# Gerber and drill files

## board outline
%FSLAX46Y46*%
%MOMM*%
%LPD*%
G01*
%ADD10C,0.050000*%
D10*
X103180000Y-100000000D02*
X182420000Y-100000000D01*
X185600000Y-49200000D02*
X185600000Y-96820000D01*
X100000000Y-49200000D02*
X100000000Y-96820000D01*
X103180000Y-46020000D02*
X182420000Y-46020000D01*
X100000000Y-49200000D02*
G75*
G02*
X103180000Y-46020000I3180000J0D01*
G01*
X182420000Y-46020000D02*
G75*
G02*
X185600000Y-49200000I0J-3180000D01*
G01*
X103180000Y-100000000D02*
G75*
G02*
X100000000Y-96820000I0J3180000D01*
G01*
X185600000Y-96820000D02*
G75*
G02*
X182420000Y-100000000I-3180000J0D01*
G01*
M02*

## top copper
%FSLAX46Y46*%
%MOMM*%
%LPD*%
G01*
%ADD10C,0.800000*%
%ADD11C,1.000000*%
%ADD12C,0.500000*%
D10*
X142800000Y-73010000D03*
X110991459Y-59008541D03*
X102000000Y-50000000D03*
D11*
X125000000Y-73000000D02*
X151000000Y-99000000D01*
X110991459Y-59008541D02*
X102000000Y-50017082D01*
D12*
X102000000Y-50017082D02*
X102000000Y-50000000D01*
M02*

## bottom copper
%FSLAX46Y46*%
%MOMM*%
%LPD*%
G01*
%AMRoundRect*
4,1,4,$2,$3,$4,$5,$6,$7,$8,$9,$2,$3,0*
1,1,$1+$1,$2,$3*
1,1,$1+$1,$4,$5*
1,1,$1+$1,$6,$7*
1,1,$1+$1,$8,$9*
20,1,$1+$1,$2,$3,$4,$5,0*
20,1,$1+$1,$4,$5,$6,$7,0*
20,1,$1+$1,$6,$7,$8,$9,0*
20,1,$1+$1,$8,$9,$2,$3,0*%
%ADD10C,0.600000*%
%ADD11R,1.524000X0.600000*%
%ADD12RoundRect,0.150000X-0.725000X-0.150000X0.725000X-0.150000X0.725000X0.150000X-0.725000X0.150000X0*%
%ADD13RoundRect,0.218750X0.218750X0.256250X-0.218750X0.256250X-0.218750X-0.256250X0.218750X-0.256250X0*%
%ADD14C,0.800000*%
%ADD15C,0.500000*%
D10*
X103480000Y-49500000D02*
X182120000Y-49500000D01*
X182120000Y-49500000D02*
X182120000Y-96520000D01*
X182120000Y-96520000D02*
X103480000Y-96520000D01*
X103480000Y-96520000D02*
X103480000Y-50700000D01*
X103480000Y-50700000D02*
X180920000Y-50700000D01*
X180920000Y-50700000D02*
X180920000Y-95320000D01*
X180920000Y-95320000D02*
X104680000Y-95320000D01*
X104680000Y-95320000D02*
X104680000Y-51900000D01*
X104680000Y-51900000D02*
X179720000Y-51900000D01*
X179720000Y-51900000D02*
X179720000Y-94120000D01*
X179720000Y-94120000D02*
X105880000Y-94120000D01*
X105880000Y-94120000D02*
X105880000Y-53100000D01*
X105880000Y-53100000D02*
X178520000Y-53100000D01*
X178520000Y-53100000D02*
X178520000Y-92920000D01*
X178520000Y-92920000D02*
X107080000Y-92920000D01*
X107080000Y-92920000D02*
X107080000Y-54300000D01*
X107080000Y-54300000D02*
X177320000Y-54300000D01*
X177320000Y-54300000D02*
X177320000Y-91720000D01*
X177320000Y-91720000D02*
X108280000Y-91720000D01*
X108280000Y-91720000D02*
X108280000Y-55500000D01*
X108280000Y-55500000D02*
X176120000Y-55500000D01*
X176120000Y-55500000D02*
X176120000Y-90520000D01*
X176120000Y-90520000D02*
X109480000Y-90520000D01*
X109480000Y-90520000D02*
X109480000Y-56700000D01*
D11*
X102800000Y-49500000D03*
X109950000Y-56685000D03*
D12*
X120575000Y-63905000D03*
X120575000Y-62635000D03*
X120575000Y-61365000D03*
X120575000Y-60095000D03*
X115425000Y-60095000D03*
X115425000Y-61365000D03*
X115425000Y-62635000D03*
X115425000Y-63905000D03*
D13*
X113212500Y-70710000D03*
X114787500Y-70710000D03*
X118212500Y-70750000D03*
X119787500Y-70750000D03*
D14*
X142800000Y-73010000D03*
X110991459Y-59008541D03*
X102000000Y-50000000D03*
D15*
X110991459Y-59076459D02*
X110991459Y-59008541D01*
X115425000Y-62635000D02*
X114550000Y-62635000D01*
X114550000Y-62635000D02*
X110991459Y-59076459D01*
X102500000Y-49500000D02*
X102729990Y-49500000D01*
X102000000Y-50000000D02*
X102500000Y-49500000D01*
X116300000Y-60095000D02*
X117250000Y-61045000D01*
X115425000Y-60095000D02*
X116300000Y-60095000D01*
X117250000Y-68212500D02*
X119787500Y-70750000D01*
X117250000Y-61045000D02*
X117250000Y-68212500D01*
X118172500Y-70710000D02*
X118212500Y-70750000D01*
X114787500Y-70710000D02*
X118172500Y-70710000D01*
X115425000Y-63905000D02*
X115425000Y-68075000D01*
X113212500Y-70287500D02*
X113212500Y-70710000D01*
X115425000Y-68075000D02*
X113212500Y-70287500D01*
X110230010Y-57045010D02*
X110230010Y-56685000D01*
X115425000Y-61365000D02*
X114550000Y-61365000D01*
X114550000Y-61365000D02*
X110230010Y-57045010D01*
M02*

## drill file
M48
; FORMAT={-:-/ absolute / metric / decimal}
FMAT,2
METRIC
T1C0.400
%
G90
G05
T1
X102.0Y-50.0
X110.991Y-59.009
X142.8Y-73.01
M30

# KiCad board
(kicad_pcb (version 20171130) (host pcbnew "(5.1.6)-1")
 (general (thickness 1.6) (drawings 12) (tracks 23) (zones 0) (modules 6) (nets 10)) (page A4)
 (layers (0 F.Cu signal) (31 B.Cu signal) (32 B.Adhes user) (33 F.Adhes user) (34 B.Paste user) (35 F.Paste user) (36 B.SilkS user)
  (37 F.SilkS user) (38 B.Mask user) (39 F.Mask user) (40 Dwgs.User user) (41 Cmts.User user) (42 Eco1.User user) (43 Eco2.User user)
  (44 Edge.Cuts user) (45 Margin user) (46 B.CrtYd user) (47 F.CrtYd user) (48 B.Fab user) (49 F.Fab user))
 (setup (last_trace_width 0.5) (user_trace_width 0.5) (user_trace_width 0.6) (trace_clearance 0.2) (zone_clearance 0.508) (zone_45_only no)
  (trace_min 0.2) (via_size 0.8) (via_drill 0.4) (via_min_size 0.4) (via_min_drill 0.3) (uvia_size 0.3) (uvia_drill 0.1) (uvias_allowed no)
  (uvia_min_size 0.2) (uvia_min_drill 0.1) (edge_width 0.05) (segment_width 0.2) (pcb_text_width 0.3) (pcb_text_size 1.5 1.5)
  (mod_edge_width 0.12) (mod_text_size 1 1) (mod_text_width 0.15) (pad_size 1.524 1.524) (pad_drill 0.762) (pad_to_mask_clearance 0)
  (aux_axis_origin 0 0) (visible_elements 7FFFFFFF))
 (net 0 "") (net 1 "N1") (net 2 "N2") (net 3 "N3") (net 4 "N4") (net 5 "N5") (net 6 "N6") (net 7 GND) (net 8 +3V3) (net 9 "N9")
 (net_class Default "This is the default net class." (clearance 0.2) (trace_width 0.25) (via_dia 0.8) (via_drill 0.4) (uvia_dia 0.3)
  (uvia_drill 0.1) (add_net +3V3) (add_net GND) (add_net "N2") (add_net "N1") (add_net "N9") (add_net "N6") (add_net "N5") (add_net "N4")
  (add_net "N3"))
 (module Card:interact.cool (layer F.Cu) (at 118 66 45)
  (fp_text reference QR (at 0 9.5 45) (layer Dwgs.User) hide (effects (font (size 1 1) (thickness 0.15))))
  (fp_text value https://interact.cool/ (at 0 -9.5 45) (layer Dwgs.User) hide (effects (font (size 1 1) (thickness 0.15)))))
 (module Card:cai (layer F.Cu) (at 150 73 270)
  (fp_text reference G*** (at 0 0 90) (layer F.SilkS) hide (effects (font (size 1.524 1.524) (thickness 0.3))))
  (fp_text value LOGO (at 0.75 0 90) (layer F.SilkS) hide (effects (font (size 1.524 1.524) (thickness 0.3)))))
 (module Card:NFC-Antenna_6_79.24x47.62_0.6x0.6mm (layer B.Cu) (at 142.8 73.01)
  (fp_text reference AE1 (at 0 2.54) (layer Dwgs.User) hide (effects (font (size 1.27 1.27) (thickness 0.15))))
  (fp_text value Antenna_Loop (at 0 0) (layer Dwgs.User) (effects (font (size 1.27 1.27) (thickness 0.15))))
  (fp_line (start -39.32 -23.51) (end 39.32 -23.51) (layer B.Cu) (width 0.6))
  (fp_line (start 39.32 -23.51) (end 39.32 23.51) (layer B.Cu) (width 0.6))
  (fp_line (start 39.32 23.51) (end -39.32 23.51) (layer B.Cu) (width 0.6))
  (fp_line (start -39.32 23.51) (end -39.32 -22.31) (layer B.Cu) (width 0.6))
  (fp_line (start -39.32 -22.31) (end 38.12 -22.31) (layer B.Cu) (width 0.6))
  (fp_line (start 38.12 -22.31) (end 38.12 22.31) (layer B.Cu) (width 0.6))
  (fp_line (start 38.12 22.31) (end -38.12 22.31) (layer B.Cu) (width 0.6))
  (fp_line (start -38.12 22.31) (end -38.12 -21.11) (layer B.Cu) (width 0.6))
  (fp_line (start -38.12 -21.11) (end 36.92 -21.11) (layer B.Cu) (width 0.6))
  (fp_line (start 36.92 -21.11) (end 36.92 21.11) (layer B.Cu) (width 0.6))
  (fp_line (start 36.92 21.11) (end -36.92 21.11) (layer B.Cu) (width 0.6))
  (fp_line (start -36.92 21.11) (end -36.92 -19.91) (layer B.Cu) (width 0.6))
  (fp_line (start -36.92 -19.91) (end 35.72 -19.91) (layer B.Cu) (width 0.6))
  (fp_line (start 35.72 -19.91) (end 35.72 19.91) (layer B.Cu) (width 0.6))
  (fp_line (start 35.72 19.91) (end -35.72 19.91) (layer B.Cu) (width 0.6))
  (fp_line (start -35.72 19.91) (end -35.72 -18.71) (layer B.Cu) (width 0.6))
  (fp_line (start -35.72 -18.71) (end 34.52 -18.71) (layer B.Cu) (width 0.6))
  (fp_line (start 34.52 -18.71) (end 34.52 18.71) (layer B.Cu) (width 0.6))
  (fp_line (start 34.52 18.71) (end -34.52 18.71) (layer B.Cu) (width 0.6))
  (fp_line (start -34.52 18.71) (end -34.52 -17.51) (layer B.Cu) (width 0.6))
  (fp_line (start -34.52 -17.51) (end 33.32 -17.51) (layer B.Cu) (width 0.6))
  (fp_line (start 33.32 -17.51) (end 33.32 17.51) (layer B.Cu) (width 0.6))
  (fp_line (start 33.32 17.51) (end -33.32 17.51) (layer B.Cu) (width 0.6))
  (fp_line (start -33.32 17.51) (end -33.32 -16.31) (layer B.Cu) (width 0.6))
  (pad 2 smd rect (at -40 -23.51) (size 1.524 0.6) (layers B.Cu) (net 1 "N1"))
  (pad 1 smd rect (at -32.85 -16.325) (size 1.524 0.6) (layers B.Cu) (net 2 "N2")))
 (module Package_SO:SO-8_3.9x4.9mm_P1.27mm (layer B.Cu) (at 118 62)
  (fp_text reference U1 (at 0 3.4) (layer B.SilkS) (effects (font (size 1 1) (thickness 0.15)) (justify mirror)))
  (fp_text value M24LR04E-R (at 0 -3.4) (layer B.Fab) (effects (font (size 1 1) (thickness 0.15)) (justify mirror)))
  (pad 8 smd roundrect (at 2.575 1.905) (size 1.75 0.6) (layers B.Cu B.Paste B.Mask) (roundrect_rratio 0.25) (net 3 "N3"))
  (pad 7 smd roundrect (at 2.575 0.635) (size 1.75 0.6) (layers B.Cu B.Paste B.Mask) (roundrect_rratio 0.25) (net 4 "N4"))
  (pad 6 smd roundrect (at 2.575 -0.635) (size 1.75 0.6) (layers B.Cu B.Paste B.Mask) (roundrect_rratio 0.25) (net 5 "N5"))
  (pad 5 smd roundrect (at 2.575 -1.905) (size 1.75 0.6) (layers B.Cu B.Paste B.Mask) (roundrect_rratio 0.25) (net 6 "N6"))
  (pad 4 smd roundrect (at -2.575 -1.905) (size 1.75 0.6) (layers B.Cu B.Paste B.Mask) (roundrect_rratio 0.25) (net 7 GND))
  (pad 3 smd roundrect (at -2.575 -0.635) (size 1.75 0.6) (layers B.Cu B.Paste B.Mask) (roundrect_rratio 0.25) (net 2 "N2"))
  (pad 2 smd roundrect (at -2.575 0.635) (size 1.75 0.6) (layers B.Cu B.Paste B.Mask) (roundrect_rratio 0.25) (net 1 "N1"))
  (pad 1 smd roundrect (at -2.575 1.905) (size 1.75 0.6) (layers B.Cu B.Paste B.Mask) (roundrect_rratio 0.25) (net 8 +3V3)))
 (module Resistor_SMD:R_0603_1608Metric (layer B.Cu) (at 114 70.71 180)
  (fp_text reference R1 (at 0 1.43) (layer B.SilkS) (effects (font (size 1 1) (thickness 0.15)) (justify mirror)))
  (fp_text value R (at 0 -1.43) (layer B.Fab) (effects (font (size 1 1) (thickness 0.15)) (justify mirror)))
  (pad 2 smd roundrect (at 0.7875 0 180) (size 0.875 0.95) (layers B.Cu B.Paste B.Mask) (roundrect_rratio 0.25) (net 8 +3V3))
  (pad 1 smd roundrect (at -0.7875 0 180) (size 0.875 0.95) (layers B.Cu B.Paste B.Mask) (roundrect_rratio 0.25) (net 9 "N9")))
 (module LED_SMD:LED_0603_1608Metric (layer B.Cu) (at 119 70.75 180)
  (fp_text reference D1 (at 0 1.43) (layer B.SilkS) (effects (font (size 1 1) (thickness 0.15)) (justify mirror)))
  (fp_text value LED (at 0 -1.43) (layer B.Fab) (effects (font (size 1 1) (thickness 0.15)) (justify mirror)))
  (pad 2 smd roundrect (at 0.7875 0 180) (size 0.875 0.95) (layers B.Cu B.Paste B.Mask) (roundrect_rratio 0.25) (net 9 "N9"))
  (pad 1 smd roundrect (at -0.7875 0 180) (size 0.875 0.95) (layers B.Cu B.Paste B.Mask) (roundrect_rratio 0.25) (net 7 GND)))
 (gr_line (start 103.18 100) (end 182.42 100) (layer Edge.Cuts) (width 0.05))
 (gr_line (start 185.6 49.2) (end 185.6 96.82) (layer Edge.Cuts) (width 0.05))
 (gr_line (start 100 49.2) (end 100 96.82) (layer Edge.Cuts) (width 0.05))
 (gr_line (start 103.18 46.02) (end 182.42 46.02) (layer Edge.Cuts) (width 0.05))
 (gr_arc (start 103.18 49.2) (end 103.18 46.02) (angle -90) (layer Edge.Cuts) (width 0.05))
 (gr_arc (start 182.42 49.2) (end 185.6 49.2) (angle -90) (layer Edge.Cuts) (width 0.05))
 (gr_arc (start 103.18 96.82) (end 100 96.82) (angle -90) (layer Edge.Cuts) (width 0.05))
 (gr_arc (start 182.42 96.82) (end 182.42 100) (angle -90) (layer Edge.Cuts) (width 0.05))
 (via (at 142.8 73.01) (size 0.8) (drill 0.4) (layers F.Cu B.Cu) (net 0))
 (segment (start 125 73) (end 151 99) (width 1) (layer F.Cu) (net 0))
 (via (at 110.991459 59.008541) (size 0.8) (drill 0.4) (layers F.Cu B.Cu) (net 1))
 (segment (start 110.991459 59.076459) (end 110.991459 59.008541) (width 0.5) (layer B.Cu) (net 1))
 (segment (start 115.425 62.635) (end 114.55 62.635) (width 0.5) (layer B.Cu) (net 1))
 (segment (start 114.55 62.635) (end 110.991459 59.076459) (width 0.5) (layer B.Cu) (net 1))
 (via (at 102 50) (size 0.8) (drill 0.4) (layers F.Cu B.Cu) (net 1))
 (segment (start 110.991459 59.008541) (end 102 50.017082) (width 1) (layer F.Cu) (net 1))
 (segment (start 102 50.017082) (end 102 50) (width 0.5) (layer F.Cu) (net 1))
 (segment (start 102.5 49.5) (end 102.72999 49.5) (width 0.5) (layer B.Cu) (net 1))
 (segment (start 102 50) (end 102.5 49.5) (width 0.5) (layer B.Cu) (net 1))
 (segment (start 116.3 60.095) (end 117.25 61.045) (width 0.5) (layer B.Cu) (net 7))
 (segment (start 115.425 60.095) (end 116.3 60.095) (width 0.5) (layer B.Cu) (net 7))
 (segment (start 117.25 68.2125) (end 119.7875 70.75) (width 0.5) (layer B.Cu) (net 7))
 (segment (start 117.25 61.045) (end 117.25 68.2125) (width 0.5) (layer B.Cu) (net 7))
 (segment (start 118.1725 70.71) (end 118.2125 70.75) (width 0.5) (layer B.Cu) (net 9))
 (segment (start 114.7875 70.71) (end 118.1725 70.71) (width 0.5) (layer B.Cu) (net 9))
 (segment (start 115.425 63.905) (end 115.425 68.075) (width 0.5) (layer B.Cu) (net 8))
 (segment (start 113.2125 70.2875) (end 113.2125 70.71) (width 0.5) (layer B.Cu) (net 8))
 (segment (start 115.425 68.075) (end 113.2125 70.2875) (width 0.5) (layer B.Cu) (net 8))
 (segment (start 110.23001 57.04501) (end 110.23001 56.685) (width 0.5) (layer B.Cu) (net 2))
 (segment (start 115.425 61.365) (end 114.55 61.365) (width 0.5) (layer B.Cu) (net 2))
 (segment (start 114.55 61.365) (end 110.23001 57.04501) (width 0.5) (layer B.Cu) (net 2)))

